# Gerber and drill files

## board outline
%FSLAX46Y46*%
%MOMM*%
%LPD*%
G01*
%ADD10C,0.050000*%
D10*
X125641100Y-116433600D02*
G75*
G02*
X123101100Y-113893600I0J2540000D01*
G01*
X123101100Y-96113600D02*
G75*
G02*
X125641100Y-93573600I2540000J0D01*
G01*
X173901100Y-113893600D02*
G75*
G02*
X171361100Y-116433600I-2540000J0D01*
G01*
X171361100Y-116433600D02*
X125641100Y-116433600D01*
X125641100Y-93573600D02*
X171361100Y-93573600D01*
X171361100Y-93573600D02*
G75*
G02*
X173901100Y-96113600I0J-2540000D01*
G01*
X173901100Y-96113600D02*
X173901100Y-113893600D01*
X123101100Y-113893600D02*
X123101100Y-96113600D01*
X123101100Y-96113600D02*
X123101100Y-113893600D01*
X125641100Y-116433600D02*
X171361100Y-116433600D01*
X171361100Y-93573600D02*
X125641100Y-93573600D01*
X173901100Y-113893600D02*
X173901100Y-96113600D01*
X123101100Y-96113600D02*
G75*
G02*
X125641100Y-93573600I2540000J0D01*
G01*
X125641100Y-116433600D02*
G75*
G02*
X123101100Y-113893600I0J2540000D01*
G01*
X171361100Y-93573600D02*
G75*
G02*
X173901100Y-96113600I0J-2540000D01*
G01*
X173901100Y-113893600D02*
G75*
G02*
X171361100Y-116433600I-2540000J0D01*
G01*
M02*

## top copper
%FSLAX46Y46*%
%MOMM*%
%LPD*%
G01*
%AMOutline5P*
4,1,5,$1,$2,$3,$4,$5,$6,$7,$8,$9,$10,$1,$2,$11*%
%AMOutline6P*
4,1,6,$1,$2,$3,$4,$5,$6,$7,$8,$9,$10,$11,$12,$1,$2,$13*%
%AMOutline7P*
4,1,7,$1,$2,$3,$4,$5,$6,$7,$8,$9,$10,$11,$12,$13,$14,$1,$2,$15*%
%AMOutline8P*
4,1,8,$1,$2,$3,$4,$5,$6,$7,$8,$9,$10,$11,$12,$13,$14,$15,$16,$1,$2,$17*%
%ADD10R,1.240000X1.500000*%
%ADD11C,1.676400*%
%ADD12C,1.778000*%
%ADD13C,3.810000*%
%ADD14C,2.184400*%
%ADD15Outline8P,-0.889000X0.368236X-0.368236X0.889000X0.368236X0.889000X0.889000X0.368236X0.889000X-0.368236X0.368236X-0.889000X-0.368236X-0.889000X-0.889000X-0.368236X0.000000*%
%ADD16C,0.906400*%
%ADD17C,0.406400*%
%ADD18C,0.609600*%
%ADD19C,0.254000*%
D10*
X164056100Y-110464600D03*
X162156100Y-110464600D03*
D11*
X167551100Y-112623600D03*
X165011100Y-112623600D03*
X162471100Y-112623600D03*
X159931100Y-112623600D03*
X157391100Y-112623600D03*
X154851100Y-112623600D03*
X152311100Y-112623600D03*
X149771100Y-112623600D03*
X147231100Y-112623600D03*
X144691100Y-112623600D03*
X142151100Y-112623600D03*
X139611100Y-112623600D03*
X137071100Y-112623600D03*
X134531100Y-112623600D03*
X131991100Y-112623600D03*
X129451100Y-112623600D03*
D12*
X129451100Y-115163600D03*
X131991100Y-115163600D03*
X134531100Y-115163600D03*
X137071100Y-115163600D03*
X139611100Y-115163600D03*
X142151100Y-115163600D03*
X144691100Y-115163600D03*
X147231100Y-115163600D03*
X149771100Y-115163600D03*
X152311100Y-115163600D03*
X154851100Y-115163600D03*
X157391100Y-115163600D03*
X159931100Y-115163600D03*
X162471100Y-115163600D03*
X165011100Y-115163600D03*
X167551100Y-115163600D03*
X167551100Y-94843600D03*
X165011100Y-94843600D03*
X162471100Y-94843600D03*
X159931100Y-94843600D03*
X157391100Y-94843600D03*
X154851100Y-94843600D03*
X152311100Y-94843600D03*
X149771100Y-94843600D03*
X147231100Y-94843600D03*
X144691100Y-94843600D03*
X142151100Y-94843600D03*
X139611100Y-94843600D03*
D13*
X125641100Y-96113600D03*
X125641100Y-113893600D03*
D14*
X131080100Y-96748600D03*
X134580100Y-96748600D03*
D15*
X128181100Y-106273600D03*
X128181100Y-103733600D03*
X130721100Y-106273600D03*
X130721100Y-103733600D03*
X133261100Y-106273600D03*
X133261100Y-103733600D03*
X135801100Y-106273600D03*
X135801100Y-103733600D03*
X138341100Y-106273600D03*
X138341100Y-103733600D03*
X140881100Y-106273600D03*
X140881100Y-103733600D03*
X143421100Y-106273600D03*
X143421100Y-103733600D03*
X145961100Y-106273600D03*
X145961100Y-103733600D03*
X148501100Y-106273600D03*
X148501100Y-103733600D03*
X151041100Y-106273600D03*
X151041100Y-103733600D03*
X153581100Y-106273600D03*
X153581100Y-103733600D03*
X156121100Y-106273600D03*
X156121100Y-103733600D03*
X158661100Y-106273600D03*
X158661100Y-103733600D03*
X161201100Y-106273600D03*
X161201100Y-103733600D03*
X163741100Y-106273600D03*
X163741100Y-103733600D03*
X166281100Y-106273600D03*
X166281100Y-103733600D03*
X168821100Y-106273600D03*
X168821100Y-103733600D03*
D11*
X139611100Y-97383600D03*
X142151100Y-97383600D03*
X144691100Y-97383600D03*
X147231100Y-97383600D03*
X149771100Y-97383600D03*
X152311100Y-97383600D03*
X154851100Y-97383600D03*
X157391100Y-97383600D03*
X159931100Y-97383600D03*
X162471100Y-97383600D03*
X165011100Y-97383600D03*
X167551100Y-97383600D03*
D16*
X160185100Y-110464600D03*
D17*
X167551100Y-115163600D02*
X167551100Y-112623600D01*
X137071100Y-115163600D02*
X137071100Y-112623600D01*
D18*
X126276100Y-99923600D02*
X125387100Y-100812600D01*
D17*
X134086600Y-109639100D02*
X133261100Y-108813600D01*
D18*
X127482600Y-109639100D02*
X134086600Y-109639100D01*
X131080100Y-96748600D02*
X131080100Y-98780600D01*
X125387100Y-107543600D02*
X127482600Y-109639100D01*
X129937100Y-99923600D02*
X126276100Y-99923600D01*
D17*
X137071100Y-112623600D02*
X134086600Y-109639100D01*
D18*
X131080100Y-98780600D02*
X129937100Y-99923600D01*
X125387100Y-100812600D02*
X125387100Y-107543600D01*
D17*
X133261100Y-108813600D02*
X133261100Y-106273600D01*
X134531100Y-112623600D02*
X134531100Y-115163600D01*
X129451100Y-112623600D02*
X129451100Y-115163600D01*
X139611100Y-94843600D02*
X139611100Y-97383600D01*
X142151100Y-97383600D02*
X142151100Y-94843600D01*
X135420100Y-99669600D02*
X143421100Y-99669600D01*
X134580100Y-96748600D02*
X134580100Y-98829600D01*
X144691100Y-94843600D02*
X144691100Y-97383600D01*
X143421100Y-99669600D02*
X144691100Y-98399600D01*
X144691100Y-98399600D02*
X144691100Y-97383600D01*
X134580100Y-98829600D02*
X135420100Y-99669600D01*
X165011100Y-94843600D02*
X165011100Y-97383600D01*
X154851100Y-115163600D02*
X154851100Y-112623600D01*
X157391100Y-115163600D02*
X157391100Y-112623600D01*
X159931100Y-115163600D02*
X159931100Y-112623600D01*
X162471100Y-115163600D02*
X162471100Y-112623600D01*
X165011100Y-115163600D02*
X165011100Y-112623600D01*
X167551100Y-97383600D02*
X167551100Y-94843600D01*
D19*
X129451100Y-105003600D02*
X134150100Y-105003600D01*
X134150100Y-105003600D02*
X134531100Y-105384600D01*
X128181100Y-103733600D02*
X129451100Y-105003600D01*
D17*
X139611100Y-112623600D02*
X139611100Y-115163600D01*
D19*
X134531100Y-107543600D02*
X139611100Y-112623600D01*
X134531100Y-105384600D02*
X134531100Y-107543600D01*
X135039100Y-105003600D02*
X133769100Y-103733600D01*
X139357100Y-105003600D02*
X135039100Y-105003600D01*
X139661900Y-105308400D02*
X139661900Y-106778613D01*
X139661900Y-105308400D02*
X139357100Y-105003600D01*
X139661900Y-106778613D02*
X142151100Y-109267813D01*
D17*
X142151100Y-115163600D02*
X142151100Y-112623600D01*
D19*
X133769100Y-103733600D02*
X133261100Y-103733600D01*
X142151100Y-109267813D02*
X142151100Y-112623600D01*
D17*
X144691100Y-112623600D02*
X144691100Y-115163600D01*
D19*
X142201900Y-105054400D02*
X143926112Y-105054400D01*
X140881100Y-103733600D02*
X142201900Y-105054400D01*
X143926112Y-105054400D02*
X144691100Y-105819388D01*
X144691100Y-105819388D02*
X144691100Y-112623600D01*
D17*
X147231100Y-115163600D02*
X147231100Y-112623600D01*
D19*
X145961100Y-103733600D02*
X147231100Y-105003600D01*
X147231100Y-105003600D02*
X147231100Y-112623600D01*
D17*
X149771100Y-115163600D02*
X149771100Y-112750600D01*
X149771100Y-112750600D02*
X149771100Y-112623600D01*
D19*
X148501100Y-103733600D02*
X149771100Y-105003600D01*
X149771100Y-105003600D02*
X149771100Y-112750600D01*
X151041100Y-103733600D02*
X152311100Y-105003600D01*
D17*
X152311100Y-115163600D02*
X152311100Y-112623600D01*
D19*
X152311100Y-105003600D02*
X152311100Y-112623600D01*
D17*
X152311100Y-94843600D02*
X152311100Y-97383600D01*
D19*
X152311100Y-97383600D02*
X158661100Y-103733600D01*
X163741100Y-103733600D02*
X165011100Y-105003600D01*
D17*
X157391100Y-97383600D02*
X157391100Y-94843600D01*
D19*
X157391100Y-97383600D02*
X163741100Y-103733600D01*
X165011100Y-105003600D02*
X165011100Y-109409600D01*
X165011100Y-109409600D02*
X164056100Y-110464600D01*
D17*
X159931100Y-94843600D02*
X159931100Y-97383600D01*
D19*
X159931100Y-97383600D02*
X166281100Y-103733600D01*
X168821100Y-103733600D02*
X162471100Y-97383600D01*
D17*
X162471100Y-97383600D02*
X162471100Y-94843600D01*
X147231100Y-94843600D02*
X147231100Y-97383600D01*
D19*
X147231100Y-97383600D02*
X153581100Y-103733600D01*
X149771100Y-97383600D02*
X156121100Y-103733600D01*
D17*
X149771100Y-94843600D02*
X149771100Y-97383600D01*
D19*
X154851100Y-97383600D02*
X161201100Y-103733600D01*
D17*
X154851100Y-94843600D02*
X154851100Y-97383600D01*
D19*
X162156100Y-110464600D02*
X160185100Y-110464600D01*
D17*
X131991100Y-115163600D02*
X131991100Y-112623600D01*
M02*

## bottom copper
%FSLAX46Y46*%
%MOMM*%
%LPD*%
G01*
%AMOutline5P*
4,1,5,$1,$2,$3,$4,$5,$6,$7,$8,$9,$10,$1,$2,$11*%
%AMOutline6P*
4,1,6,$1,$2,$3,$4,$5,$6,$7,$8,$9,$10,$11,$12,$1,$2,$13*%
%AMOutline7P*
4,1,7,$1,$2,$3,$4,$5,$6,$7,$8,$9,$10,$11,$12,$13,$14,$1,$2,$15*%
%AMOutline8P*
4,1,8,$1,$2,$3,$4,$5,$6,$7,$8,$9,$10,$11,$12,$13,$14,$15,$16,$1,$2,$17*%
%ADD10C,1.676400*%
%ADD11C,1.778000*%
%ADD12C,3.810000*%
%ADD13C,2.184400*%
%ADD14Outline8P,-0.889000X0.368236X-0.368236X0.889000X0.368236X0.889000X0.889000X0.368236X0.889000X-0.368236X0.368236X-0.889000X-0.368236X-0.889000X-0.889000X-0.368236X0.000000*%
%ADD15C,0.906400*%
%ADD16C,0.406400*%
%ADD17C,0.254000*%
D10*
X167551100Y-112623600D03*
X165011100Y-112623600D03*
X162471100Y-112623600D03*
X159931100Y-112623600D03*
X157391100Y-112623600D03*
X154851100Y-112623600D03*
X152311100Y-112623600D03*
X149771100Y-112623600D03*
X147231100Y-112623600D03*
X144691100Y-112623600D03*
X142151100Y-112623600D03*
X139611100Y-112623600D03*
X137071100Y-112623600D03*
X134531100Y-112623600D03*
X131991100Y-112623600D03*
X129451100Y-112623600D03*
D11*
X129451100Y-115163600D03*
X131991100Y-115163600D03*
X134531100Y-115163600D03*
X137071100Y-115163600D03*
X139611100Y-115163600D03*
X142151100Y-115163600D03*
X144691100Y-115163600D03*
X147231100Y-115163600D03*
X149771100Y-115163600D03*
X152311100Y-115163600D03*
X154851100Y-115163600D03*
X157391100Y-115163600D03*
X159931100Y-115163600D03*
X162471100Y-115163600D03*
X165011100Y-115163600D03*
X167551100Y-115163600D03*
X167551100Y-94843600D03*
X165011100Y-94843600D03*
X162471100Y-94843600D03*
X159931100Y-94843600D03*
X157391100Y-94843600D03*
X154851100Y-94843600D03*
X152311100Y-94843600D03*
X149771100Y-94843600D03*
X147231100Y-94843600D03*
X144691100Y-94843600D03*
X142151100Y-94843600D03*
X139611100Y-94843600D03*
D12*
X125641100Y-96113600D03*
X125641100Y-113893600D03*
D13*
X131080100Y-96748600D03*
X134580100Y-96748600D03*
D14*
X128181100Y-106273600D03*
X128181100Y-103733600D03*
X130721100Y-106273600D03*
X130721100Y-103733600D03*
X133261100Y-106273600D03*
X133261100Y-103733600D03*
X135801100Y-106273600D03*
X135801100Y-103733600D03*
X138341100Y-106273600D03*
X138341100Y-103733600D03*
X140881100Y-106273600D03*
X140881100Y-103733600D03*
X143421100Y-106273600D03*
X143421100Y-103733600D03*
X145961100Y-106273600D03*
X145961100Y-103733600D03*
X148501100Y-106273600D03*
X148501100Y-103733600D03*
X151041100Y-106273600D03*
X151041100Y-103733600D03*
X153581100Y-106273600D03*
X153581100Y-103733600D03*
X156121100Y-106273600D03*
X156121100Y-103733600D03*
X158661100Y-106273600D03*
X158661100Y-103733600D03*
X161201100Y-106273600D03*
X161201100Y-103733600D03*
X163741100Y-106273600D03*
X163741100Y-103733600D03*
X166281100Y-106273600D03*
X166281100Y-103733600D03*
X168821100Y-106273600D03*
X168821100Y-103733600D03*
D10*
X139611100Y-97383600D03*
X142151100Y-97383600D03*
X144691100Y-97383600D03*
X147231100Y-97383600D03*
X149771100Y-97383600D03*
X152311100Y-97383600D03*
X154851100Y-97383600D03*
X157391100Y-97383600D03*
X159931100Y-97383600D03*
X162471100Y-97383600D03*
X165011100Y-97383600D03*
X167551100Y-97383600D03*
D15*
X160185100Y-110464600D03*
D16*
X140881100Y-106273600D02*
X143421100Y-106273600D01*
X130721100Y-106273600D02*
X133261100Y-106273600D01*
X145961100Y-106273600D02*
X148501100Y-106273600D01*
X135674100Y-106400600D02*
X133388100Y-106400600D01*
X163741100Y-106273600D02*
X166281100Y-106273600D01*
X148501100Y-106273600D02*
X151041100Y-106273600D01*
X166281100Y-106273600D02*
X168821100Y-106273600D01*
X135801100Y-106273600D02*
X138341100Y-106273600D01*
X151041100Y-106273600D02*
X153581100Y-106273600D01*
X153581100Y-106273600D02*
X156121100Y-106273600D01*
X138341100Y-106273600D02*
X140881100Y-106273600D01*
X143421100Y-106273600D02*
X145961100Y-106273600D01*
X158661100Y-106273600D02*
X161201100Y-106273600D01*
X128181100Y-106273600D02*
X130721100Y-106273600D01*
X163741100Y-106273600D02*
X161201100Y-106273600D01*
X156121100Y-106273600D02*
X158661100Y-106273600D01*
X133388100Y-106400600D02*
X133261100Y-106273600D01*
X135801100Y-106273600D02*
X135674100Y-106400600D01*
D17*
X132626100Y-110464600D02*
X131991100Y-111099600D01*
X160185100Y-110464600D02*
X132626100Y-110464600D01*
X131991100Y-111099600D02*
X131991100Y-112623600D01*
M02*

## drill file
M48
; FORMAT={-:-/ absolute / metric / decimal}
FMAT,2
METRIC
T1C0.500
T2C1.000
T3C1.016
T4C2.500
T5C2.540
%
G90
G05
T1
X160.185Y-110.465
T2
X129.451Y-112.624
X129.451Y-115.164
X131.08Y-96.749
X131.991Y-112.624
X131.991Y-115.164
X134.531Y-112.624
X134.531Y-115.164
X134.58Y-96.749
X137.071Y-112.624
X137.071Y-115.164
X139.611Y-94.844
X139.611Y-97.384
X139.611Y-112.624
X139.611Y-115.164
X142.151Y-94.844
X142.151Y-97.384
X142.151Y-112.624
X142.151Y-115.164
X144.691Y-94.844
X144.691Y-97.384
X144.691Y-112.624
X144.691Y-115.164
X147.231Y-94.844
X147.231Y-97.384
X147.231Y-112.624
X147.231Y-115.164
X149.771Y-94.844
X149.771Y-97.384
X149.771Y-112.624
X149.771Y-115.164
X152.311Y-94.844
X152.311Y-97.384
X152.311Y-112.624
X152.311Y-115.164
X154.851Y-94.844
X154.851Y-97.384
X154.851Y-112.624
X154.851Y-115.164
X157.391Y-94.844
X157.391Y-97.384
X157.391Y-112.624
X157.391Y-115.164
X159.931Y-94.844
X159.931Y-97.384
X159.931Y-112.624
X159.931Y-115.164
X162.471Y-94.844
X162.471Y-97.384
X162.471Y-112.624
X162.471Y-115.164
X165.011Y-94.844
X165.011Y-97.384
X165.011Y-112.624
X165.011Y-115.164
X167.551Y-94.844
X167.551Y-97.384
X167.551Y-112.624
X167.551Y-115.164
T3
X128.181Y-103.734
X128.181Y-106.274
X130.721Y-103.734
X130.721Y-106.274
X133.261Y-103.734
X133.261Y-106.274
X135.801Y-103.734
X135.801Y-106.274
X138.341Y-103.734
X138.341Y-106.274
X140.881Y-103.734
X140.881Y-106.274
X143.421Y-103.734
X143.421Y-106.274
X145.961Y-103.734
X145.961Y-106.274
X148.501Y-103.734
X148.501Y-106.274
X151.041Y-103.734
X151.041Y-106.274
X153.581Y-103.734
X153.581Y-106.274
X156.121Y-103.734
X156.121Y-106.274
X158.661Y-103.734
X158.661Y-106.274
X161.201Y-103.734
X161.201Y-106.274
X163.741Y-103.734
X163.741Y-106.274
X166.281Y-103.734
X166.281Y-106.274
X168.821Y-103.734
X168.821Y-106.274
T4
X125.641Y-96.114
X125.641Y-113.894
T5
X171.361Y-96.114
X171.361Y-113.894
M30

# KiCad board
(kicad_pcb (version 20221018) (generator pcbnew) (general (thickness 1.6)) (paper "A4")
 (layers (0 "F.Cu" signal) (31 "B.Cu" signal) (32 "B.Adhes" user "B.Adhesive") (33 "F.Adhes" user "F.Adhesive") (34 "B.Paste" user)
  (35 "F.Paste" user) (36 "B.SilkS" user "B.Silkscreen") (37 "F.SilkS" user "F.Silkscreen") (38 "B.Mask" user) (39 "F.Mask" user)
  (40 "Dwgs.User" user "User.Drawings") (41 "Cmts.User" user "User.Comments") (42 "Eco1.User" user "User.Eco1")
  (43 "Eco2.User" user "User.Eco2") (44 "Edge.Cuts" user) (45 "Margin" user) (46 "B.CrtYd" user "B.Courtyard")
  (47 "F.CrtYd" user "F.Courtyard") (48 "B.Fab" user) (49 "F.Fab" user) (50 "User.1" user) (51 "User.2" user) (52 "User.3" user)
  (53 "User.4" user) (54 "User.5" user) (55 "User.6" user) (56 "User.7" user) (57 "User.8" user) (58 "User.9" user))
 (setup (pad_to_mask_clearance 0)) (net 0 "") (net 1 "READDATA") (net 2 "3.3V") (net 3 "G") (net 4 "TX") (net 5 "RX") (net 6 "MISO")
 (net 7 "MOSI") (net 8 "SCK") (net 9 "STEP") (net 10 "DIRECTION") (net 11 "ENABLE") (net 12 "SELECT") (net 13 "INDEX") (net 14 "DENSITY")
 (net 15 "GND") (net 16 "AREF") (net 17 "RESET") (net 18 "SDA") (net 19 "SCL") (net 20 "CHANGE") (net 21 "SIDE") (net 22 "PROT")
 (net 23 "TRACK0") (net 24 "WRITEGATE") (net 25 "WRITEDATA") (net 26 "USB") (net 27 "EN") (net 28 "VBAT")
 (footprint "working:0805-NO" (layer "F.Cu") (at 163.1061 110.4646 180)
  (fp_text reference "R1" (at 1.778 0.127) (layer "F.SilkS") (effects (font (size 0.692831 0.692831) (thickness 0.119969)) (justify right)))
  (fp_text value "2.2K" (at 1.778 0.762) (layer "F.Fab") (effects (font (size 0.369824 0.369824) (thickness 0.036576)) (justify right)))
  (pad "1" smd rect (at -0.95 0 180) (size 1.24 1.5) (layers "F.Cu" "F.Paste" "F.Mask") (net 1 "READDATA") (solder_mask_margin 0.0508)
   (thermal_bridge_angle 45))
  (pad "2" smd rect (at 0.95 0 180) (size 1.24 1.5) (layers "F.Cu" "F.Paste" "F.Mask") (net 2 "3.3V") (solder_mask_margin 0.0508)
   (thermal_bridge_angle 45)))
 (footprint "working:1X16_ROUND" (layer "F.Cu") (at 148.5011 112.6236 180)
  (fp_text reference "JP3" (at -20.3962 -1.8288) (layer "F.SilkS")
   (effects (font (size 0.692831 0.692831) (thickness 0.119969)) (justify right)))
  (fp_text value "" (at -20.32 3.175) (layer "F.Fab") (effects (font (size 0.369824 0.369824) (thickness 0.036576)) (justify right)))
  (pad "1" thru_hole circle (at -19.05 0 270) (size 1.6764 1.6764) (drill 1) (layers "*.Cu" "*.Mask") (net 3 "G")
   (solder_mask_margin 0.0508))
  (pad "2" thru_hole circle (at -16.51 0 270) (size 1.6764 1.6764) (drill 1) (layers "*.Cu" "*.Mask") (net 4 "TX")
   (solder_mask_margin 0.0508))
  (pad "3" thru_hole circle (at -13.97 0 270) (size 1.6764 1.6764) (drill 1) (layers "*.Cu" "*.Mask") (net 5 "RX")
   (solder_mask_margin 0.0508))
  (pad "4" thru_hole circle (at -11.43 0 270) (size 1.6764 1.6764) (drill 1) (layers "*.Cu" "*.Mask") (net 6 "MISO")
   (solder_mask_margin 0.0508))
  (pad "5" thru_hole circle (at -8.89 0 270) (size 1.6764 1.6764) (drill 1) (layers "*.Cu" "*.Mask") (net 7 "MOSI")
   (solder_mask_margin 0.0508))
  (pad "6" thru_hole circle (at -6.35 0 270) (size 1.6764 1.6764) (drill 1) (layers "*.Cu" "*.Mask") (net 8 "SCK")
   (solder_mask_margin 0.0508))
  (pad "7" thru_hole circle (at -3.81 0 270) (size 1.6764 1.6764) (drill 1) (layers "*.Cu" "*.Mask") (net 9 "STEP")
   (solder_mask_margin 0.0508))
  (pad "8" thru_hole circle (at -1.27 0 270) (size 1.6764 1.6764) (drill 1) (layers "*.Cu" "*.Mask") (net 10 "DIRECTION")
   (solder_mask_margin 0.0508))
  (pad "9" thru_hole circle (at 1.27 0 270) (size 1.6764 1.6764) (drill 1) (layers "*.Cu" "*.Mask") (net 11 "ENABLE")
   (solder_mask_margin 0.0508))
  (pad "10" thru_hole circle (at 3.81 0 270) (size 1.6764 1.6764) (drill 1) (layers "*.Cu" "*.Mask") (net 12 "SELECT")
   (solder_mask_margin 0.0508))
  (pad "11" thru_hole circle (at 6.35 0 270) (size 1.6764 1.6764) (drill 1) (layers "*.Cu" "*.Mask") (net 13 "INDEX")
   (solder_mask_margin 0.0508))
  (pad "12" thru_hole circle (at 8.89 0 270) (size 1.6764 1.6764) (drill 1) (layers "*.Cu" "*.Mask") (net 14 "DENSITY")
   (solder_mask_margin 0.0508))
  (pad "13" thru_hole circle (at 11.43 0 270) (size 1.6764 1.6764) (drill 1) (layers "*.Cu" "*.Mask") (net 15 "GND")
   (solder_mask_margin 0.0508))
  (pad "14" thru_hole circle (at 13.97 0 270) (size 1.6764 1.6764) (drill 1) (layers "*.Cu" "*.Mask") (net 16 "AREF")
   (solder_mask_margin 0.0508))
  (pad "15" thru_hole circle (at 16.51 0 270) (size 1.6764 1.6764) (drill 1) (layers "*.Cu" "*.Mask") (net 2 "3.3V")
   (solder_mask_margin 0.0508))
  (pad "16" thru_hole circle (at 19.05 0 270) (size 1.6764 1.6764) (drill 1) (layers "*.Cu" "*.Mask") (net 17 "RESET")
   (solder_mask_margin 0.0508)))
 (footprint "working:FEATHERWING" (layer "F.Cu") (at 123.1011 116.4336)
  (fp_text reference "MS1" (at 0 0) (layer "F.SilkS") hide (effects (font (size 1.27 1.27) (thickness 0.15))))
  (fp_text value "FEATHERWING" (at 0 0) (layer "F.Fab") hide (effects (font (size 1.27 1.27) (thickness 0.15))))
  (fp_line (start 0 -20.32) (end 0 -2.54) (stroke (width 0.05) (type solid)) (layer "Edge.Cuts"))
  (fp_line (start 2.54 0) (end 48.26 0) (stroke (width 0.05) (type solid)) (layer "Edge.Cuts"))
  (fp_line (start 48.26 -22.86) (end 2.54 -22.86) (stroke (width 0.05) (type solid)) (layer "Edge.Cuts"))
  (fp_line (start 50.8 -2.54) (end 50.8 -20.32) (stroke (width 0.05) (type solid)) (layer "Edge.Cuts"))
  (fp_arc (start 0 -20.32) (mid 0.743949 -22.116051) (end 2.54 -22.86) (stroke (width 0.05) (type solid)) (layer "Edge.Cuts"))
  (fp_arc (start 2.54 0) (mid 0.743949 -0.743949) (end 0 -2.54) (stroke (width 0.05) (type solid)) (layer "Edge.Cuts"))
  (fp_arc (start 48.26 -22.86) (mid 50.056051 -22.116051) (end 50.8 -20.32) (stroke (width 0.05) (type solid)) (layer "Edge.Cuts"))
  (fp_arc (start 50.8 -2.54) (mid 50.056051 -0.743949) (end 48.26 0) (stroke (width 0.05) (type solid)) (layer "Edge.Cuts"))
  (pad "" np_thru_hole circle (at 48.26 -20.32) (size 2.54 2.54) (drill 2.54) (layers "*.Cu" "*.Mask"))
  (pad "" np_thru_hole circle (at 48.26 -2.54) (size 2.54 2.54) (drill 2.54) (layers "*.Cu" "*.Mask"))
  (pad "1" thru_hole circle (at 6.35 -1.27) (size 1.778 1.778) (drill 1) (layers "*.Cu" "*.Mask") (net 17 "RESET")
   (solder_mask_margin 0.0508))
  (pad "2" thru_hole circle (at 8.89 -1.27) (size 1.778 1.778) (drill 1) (layers "*.Cu" "*.Mask") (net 2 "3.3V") (solder_mask_margin 0.0508))
  (pad "3" thru_hole circle (at 11.43 -1.27) (size 1.778 1.778) (drill 1) (layers "*.Cu" "*.Mask") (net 16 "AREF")
   (solder_mask_margin 0.0508))
  (pad "4" thru_hole circle (at 13.97 -1.27) (size 1.778 1.778) (drill 1) (layers "*.Cu" "*.Mask") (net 15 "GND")
   (solder_mask_margin 0.0508))
  (pad "5" thru_hole circle (at 16.51 -1.27) (size 1.778 1.778) (drill 1) (layers "*.Cu" "*.Mask") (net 14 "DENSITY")
   (solder_mask_margin 0.0508))
  (pad "6" thru_hole circle (at 19.05 -1.27) (size 1.778 1.778) (drill 1) (layers "*.Cu" "*.Mask") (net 13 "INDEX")
   (solder_mask_margin 0.0508))
  (pad "7" thru_hole circle (at 21.59 -1.27) (size 1.778 1.778) (drill 1) (layers "*.Cu" "*.Mask") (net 12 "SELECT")
   (solder_mask_margin 0.0508))
  (pad "8" thru_hole circle (at 24.13 -1.27) (size 1.778 1.778) (drill 1) (layers "*.Cu" "*.Mask") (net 11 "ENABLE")
   (solder_mask_margin 0.0508))
  (pad "9" thru_hole circle (at 26.67 -1.27) (size 1.778 1.778) (drill 1) (layers "*.Cu" "*.Mask") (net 10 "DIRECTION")
   (solder_mask_margin 0.0508))
  (pad "10" thru_hole circle (at 29.21 -1.27) (size 1.778 1.778) (drill 1) (layers "*.Cu" "*.Mask") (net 9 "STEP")
   (solder_mask_margin 0.0508))
  (pad "11" thru_hole circle (at 31.75 -1.27) (size 1.778 1.778) (drill 1) (layers "*.Cu" "*.Mask") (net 8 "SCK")
   (solder_mask_margin 0.0508))
  (pad "12" thru_hole circle (at 34.29 -1.27) (size 1.778 1.778) (drill 1) (layers "*.Cu" "*.Mask") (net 7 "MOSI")
   (solder_mask_margin 0.0508))
  (pad "13" thru_hole circle (at 36.83 -1.27) (size 1.778 1.778) (drill 1) (layers "*.Cu" "*.Mask") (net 6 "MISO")
   (solder_mask_margin 0.0508))
  (pad "14" thru_hole circle (at 39.37 -1.27) (size 1.778 1.778) (drill 1) (layers "*.Cu" "*.Mask") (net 5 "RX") (solder_mask_margin 0.0508))
  (pad "15" thru_hole circle (at 41.91 -1.27) (size 1.778 1.778) (drill 1) (layers "*.Cu" "*.Mask") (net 4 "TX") (solder_mask_margin 0.0508))
  (pad "16" thru_hole circle (at 44.45 -1.27) (size 1.778 1.778) (drill 1) (layers "*.Cu" "*.Mask") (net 3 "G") (solder_mask_margin 0.0508))
  (pad "17" thru_hole circle (at 44.45 -21.59) (size 1.778 1.778) (drill 1) (layers "*.Cu" "*.Mask") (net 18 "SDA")
   (solder_mask_margin 0.0508))
  (pad "18" thru_hole circle (at 41.91 -21.59) (size 1.778 1.778) (drill 1) (layers "*.Cu" "*.Mask") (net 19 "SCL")
   (solder_mask_margin 0.0508))
  (pad "19" thru_hole circle (at 39.37 -21.59) (size 1.778 1.778) (drill 1) (layers "*.Cu" "*.Mask") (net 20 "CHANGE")
   (solder_mask_margin 0.0508))
  (pad "20" thru_hole circle (at 36.83 -21.59) (size 1.778 1.778) (drill 1) (layers "*.Cu" "*.Mask") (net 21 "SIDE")
   (solder_mask_margin 0.0508))
  (pad "21" thru_hole circle (at 34.29 -21.59) (size 1.778 1.778) (drill 1) (layers "*.Cu" "*.Mask") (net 1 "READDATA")
   (solder_mask_margin 0.0508))
  (pad "22" thru_hole circle (at 31.75 -21.59) (size 1.778 1.778) (drill 1) (layers "*.Cu" "*.Mask") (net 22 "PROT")
   (solder_mask_margin 0.0508))
  (pad "23" thru_hole circle (at 29.21 -21.59) (size 1.778 1.778) (drill 1) (layers "*.Cu" "*.Mask") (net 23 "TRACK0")
   (solder_mask_margin 0.0508))
  (pad "24" thru_hole circle (at 26.67 -21.59) (size 1.778 1.778) (drill 1) (layers "*.Cu" "*.Mask") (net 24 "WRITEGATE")
   (solder_mask_margin 0.0508))
  (pad "25" thru_hole circle (at 24.13 -21.59) (size 1.778 1.778) (drill 1) (layers "*.Cu" "*.Mask") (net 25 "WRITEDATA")
   (solder_mask_margin 0.0508))
  (pad "26" thru_hole circle (at 21.59 -21.59) (size 1.778 1.778) (drill 1) (layers "*.Cu" "*.Mask") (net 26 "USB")
   (solder_mask_margin 0.0508))
  (pad "27" thru_hole circle (at 19.05 -21.59) (size 1.778 1.778) (drill 1) (layers "*.Cu" "*.Mask") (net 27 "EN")
   (solder_mask_margin 0.0508))
  (pad "28" thru_hole circle (at 16.51 -21.59) (size 1.778 1.778) (drill 1) (layers "*.Cu" "*.Mask") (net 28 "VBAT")
   (solder_mask_margin 0.0508))
  (pad "P$1" thru_hole circle (at 2.54 -20.32) (size 3.81 3.81) (drill 2.5) (layers "*.Cu" "*.Mask") (solder_mask_margin 0.0508))
  (pad "P$2" thru_hole circle (at 2.54 -2.54) (size 3.81 3.81) (drill 2.5) (layers "*.Cu" "*.Mask") (solder_mask_margin 0.0508)))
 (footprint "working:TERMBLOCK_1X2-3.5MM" (layer "F.Cu") (at 132.8801 96.7486 180)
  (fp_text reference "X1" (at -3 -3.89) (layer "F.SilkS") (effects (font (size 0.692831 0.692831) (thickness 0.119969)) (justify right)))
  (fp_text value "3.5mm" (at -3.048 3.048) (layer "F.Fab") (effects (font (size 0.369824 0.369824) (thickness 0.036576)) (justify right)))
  (pad "1" thru_hole circle (at 1.8 0 180) (size 2.1844 2.1844) (drill 1) (layers "*.Cu" "*.Mask") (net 15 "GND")
   (solder_mask_margin 0.0508))
  (pad "2" thru_hole circle (at -1.7 0 180) (size 2.1844 2.1844) (drill 1) (layers "*.Cu" "*.Mask") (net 26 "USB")
   (solder_mask_margin 0.0508)))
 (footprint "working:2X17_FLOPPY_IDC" (layer "F.Cu") (at 148.5011 105.0036 90)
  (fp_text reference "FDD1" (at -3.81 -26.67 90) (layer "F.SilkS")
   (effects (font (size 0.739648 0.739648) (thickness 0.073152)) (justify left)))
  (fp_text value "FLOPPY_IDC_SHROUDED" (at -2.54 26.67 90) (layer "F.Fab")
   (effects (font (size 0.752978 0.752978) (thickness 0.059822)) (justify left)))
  (pad "1" thru_hole roundrect (at -1.27 -20.32) (size 1.778 1.778) (drill 1.016) (layers "*.Cu" "*.Mask") (roundrect_rratio 0.25)
   (chamfer_ratio 0.2928932188) (chamfer top_left top_right bottom_left bottom_right) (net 15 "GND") (solder_mask_margin 0.0508)
   (thermal_bridge_angle 45))
  (pad "2" thru_hole roundrect (at 1.27 -20.32) (size 1.778 1.778) (drill 1.016) (layers "*.Cu" "*.Mask") (roundrect_rratio 0.25)
   (chamfer_ratio 0.2928932188) (chamfer top_left top_right bottom_left bottom_right) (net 14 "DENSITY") (solder_mask_margin 0.0508)
   (thermal_bridge_angle 45))
  (pad "3" thru_hole roundrect (at -1.27 -17.78) (size 1.778 1.778) (drill 1.016) (layers "*.Cu" "*.Mask") (roundrect_rratio 0.25)
   (chamfer_ratio 0.2928932188) (chamfer top_left top_right bottom_left bottom_right) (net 15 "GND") (solder_mask_margin 0.0508)
   (thermal_bridge_angle 45))
  (pad "4" thru_hole roundrect (at 1.27 -17.78) (size 1.778 1.778) (drill 1.016) (layers "*.Cu" "*.Mask") (roundrect_rratio 0.25)
   (chamfer_ratio 0.2928932188) (chamfer top_left top_right bottom_left bottom_right) (solder_mask_margin 0.0508) (thermal_bridge_angle 45))
  (pad "5" thru_hole roundrect (at -1.27 -15.24) (size 1.778 1.778) (drill 1.016) (layers "*.Cu" "*.Mask") (roundrect_rratio 0.25)
   (chamfer_ratio 0.2928932188) (chamfer top_left top_right bottom_left bottom_right) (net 15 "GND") (solder_mask_margin 0.0508)
   (thermal_bridge_angle 45))
  (pad "6" thru_hole roundrect (at 1.27 -15.24) (size 1.778 1.778) (drill 1.016) (layers "*.Cu" "*.Mask") (roundrect_rratio 0.25)
   (chamfer_ratio 0.2928932188) (chamfer top_left top_right bottom_left bottom_right) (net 13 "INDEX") (solder_mask_margin 0.0508)
   (thermal_bridge_angle 45))
  (pad "7" thru_hole roundrect (at -1.27 -12.7) (size 1.778 1.778) (drill 1.016) (layers "*.Cu" "*.Mask") (roundrect_rratio 0.25)
   (chamfer_ratio 0.2928932188) (chamfer top_left top_right bottom_left bottom_right) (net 15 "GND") (solder_mask_margin 0.0508)
   (thermal_bridge_angle 45))
  (pad "8" thru_hole roundrect (at 1.27 -12.7) (size 1.778 1.778) (drill 1.016) (layers "*.Cu" "*.Mask") (roundrect_rratio 0.25)
   (chamfer_ratio 0.2928932188) (chamfer top_left top_right bottom_left bottom_right) (solder_mask_margin 0.0508) (thermal_bridge_angle 45))
  (pad "9" thru_hole roundrect (at -1.27 -10.16) (size 1.778 1.778) (drill 1.016) (layers "*.Cu" "*.Mask") (roundrect_rratio 0.25)
   (chamfer_ratio 0.2928932188) (chamfer top_left top_right bottom_left bottom_right) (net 15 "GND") (solder_mask_margin 0.0508)
   (thermal_bridge_angle 45))
  (pad "10" thru_hole roundrect (at 1.27 -10.16) (size 1.778 1.778) (drill 1.016) (layers "*.Cu" "*.Mask") (roundrect_rratio 0.25)
   (chamfer_ratio 0.2928932188) (chamfer top_left top_right bottom_left bottom_right) (solder_mask_margin 0.0508) (thermal_bridge_angle 45))
  (pad "11" thru_hole roundrect (at -1.27 -7.62) (size 1.778 1.778) (drill 1.016) (layers "*.Cu" "*.Mask") (roundrect_rratio 0.25)
   (chamfer_ratio 0.2928932188) (chamfer top_left top_right bottom_left bottom_right) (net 15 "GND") (solder_mask_margin 0.0508)
   (thermal_bridge_angle 45))
  (pad "12" thru_hole roundrect (at 1.27 -7.62) (size 1.778 1.778) (drill 1.016) (layers "*.Cu" "*.Mask") (roundrect_rratio 0.25)
   (chamfer_ratio 0.2928932188) (chamfer top_left top_right bottom_left bottom_right) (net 12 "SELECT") (solder_mask_margin 0.0508)
   (thermal_bridge_angle 45))
  (pad "13" thru_hole roundrect (at -1.27 -5.08) (size 1.778 1.778) (drill 1.016) (layers "*.Cu" "*.Mask") (roundrect_rratio 0.25)
   (chamfer_ratio 0.2928932188) (chamfer top_left top_right bottom_left bottom_right) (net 15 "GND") (solder_mask_margin 0.0508)
   (thermal_bridge_angle 45))
  (pad "14" thru_hole roundrect (at 1.27 -5.08) (size 1.778 1.778) (drill 1.016) (layers "*.Cu" "*.Mask") (roundrect_rratio 0.25)
   (chamfer_ratio 0.2928932188) (chamfer top_left top_right bottom_left bottom_right) (solder_mask_margin 0.0508) (thermal_bridge_angle 45))
  (pad "15" thru_hole roundrect (at -1.27 -2.54) (size 1.778 1.778) (drill 1.016) (layers "*.Cu" "*.Mask") (roundrect_rratio 0.25)
   (chamfer_ratio 0.2928932188) (chamfer top_left top_right bottom_left bottom_right) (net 15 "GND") (solder_mask_margin 0.0508)
   (thermal_bridge_angle 45))
  (pad "16" thru_hole roundrect (at 1.27 -2.54) (size 1.778 1.778) (drill 1.016) (layers "*.Cu" "*.Mask") (roundrect_rratio 0.25)
   (chamfer_ratio 0.2928932188) (chamfer top_left top_right bottom_left bottom_right) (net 11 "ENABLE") (solder_mask_margin 0.0508)
   (thermal_bridge_angle 45))
  (pad "17" thru_hole roundrect (at -1.27 0) (size 1.778 1.778) (drill 1.016) (layers "*.Cu" "*.Mask") (roundrect_rratio 0.25)
   (chamfer_ratio 0.2928932188) (chamfer top_left top_right bottom_left bottom_right) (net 15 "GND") (solder_mask_margin 0.0508)
   (thermal_bridge_angle 45))
  (pad "18" thru_hole roundrect (at 1.27 0) (size 1.778 1.778) (drill 1.016) (layers "*.Cu" "*.Mask") (roundrect_rratio 0.25)
   (chamfer_ratio 0.2928932188) (chamfer top_left top_right bottom_left bottom_right) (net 10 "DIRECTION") (solder_mask_margin 0.0508)
   (thermal_bridge_angle 45))
  (pad "19" thru_hole roundrect (at -1.27 2.54) (size 1.778 1.778) (drill 1.016) (layers "*.Cu" "*.Mask") (roundrect_rratio 0.25)
   (chamfer_ratio 0.2928932188) (chamfer top_left top_right bottom_left bottom_right) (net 15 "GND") (solder_mask_margin 0.0508)
   (thermal_bridge_angle 45))
  (pad "20" thru_hole roundrect (at 1.27 2.54) (size 1.778 1.778) (drill 1.016) (layers "*.Cu" "*.Mask") (roundrect_rratio 0.25)
   (chamfer_ratio 0.2928932188) (chamfer top_left top_right bottom_left bottom_right) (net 9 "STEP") (solder_mask_margin 0.0508)
   (thermal_bridge_angle 45))
  (pad "21" thru_hole roundrect (at -1.27 5.08) (size 1.778 1.778) (drill 1.016) (layers "*.Cu" "*.Mask") (roundrect_rratio 0.25)
   (chamfer_ratio 0.2928932188) (chamfer top_left top_right bottom_left bottom_right) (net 15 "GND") (solder_mask_margin 0.0508)
   (thermal_bridge_angle 45))
  (pad "22" thru_hole roundrect (at 1.27 5.08) (size 1.778 1.778) (drill 1.016) (layers "*.Cu" "*.Mask") (roundrect_rratio 0.25)
   (chamfer_ratio 0.2928932188) (chamfer top_left top_right bottom_left bottom_right) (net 25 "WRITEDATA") (solder_mask_margin 0.0508)
   (thermal_bridge_angle 45))
  (pad "23" thru_hole roundrect (at -1.27 7.62) (size 1.778 1.778) (drill 1.016) (layers "*.Cu" "*.Mask") (roundrect_rratio 0.25)
   (chamfer_ratio 0.2928932188) (chamfer top_left top_right bottom_left bottom_right) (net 15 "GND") (solder_mask_margin 0.0508)
   (thermal_bridge_angle 45))
  (pad "24" thru_hole roundrect (at 1.27 7.62) (size 1.778 1.778) (drill 1.016) (layers "*.Cu" "*.Mask") (roundrect_rratio 0.25)
   (chamfer_ratio 0.2928932188) (chamfer top_left top_right bottom_left bottom_right) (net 24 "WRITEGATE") (solder_mask_margin 0.0508)
   (thermal_bridge_angle 45))
  (pad "25" thru_hole roundrect (at -1.27 10.16) (size 1.778 1.778) (drill 1.016) (layers "*.Cu" "*.Mask") (roundrect_rratio 0.25)
   (chamfer_ratio 0.2928932188) (chamfer top_left top_right bottom_left bottom_right) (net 15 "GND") (solder_mask_margin 0.0508)
   (thermal_bridge_angle 45))
  (pad "26" thru_hole roundrect (at 1.27 10.16) (size 1.778 1.778) (drill 1.016) (layers "*.Cu" "*.Mask") (roundrect_rratio 0.25)
   (chamfer_ratio 0.2928932188) (chamfer top_left top_right bottom_left bottom_right) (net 23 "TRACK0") (solder_mask_margin 0.0508)
   (thermal_bridge_angle 45))
  (pad "27" thru_hole roundrect (at -1.27 12.7) (size 1.778 1.778) (drill 1.016) (layers "*.Cu" "*.Mask") (roundrect_rratio 0.25)
   (chamfer_ratio 0.2928932188) (chamfer top_left top_right bottom_left bottom_right) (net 15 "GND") (solder_mask_margin 0.0508)
   (thermal_bridge_angle 45))
  (pad "28" thru_hole roundrect (at 1.27 12.7) (size 1.778 1.778) (drill 1.016) (layers "*.Cu" "*.Mask") (roundrect_rratio 0.25)
   (chamfer_ratio 0.2928932188) (chamfer top_left top_right bottom_left bottom_right) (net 22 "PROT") (solder_mask_margin 0.0508)
   (thermal_bridge_angle 45))
  (pad "29" thru_hole roundrect (at -1.27 15.24) (size 1.778 1.778) (drill 1.016) (layers "*.Cu" "*.Mask") (roundrect_rratio 0.25)
   (chamfer_ratio 0.2928932188) (chamfer top_left top_right bottom_left bottom_right) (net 15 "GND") (solder_mask_margin 0.0508)
   (thermal_bridge_angle 45))
  (pad "30" thru_hole roundrect (at 1.27 15.24) (size 1.778 1.778) (drill 1.016) (layers "*.Cu" "*.Mask") (roundrect_rratio 0.25)
   (chamfer_ratio 0.2928932188) (chamfer top_left top_right bottom_left bottom_right) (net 1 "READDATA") (solder_mask_margin 0.0508)
   (thermal_bridge_angle 45))
  (pad "31" thru_hole roundrect (at -1.27 17.78) (size 1.778 1.778) (drill 1.016) (layers "*.Cu" "*.Mask") (roundrect_rratio 0.25)
   (chamfer_ratio 0.2928932188) (chamfer top_left top_right bottom_left bottom_right) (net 15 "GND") (solder_mask_margin 0.0508)
   (thermal_bridge_angle 45))
  (pad "32" thru_hole roundrect (at 1.27 17.78) (size 1.778 1.778) (drill 1.016) (layers "*.Cu" "*.Mask") (roundrect_rratio 0.25)
   (chamfer_ratio 0.2928932188) (chamfer top_left top_right bottom_left bottom_right) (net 21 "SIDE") (solder_mask_margin 0.0508)
   (thermal_bridge_angle 45))
  (pad "33" thru_hole roundrect (at -1.27 20.32) (size 1.778 1.778) (drill 1.016) (layers "*.Cu" "*.Mask") (roundrect_rratio 0.25)
   (chamfer_ratio 0.2928932188) (chamfer top_left top_right bottom_left bottom_right) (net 15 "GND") (solder_mask_margin 0.0508)
   (thermal_bridge_angle 45))
  (pad "34" thru_hole roundrect (at 1.27 20.32) (size 1.778 1.778) (drill 1.016) (layers "*.Cu" "*.Mask") (roundrect_rratio 0.25)
   (chamfer_ratio 0.2928932188) (chamfer top_left top_right bottom_left bottom_right) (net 20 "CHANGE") (solder_mask_margin 0.0508)
   (thermal_bridge_angle 45)))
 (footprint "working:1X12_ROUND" (layer "F.Cu") (at 153.5811 97.3836)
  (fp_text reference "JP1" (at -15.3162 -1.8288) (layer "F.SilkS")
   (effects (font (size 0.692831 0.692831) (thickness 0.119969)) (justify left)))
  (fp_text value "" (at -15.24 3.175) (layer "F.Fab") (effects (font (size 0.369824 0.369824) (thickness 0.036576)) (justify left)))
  (pad "1" thru_hole circle (at -13.97 0 90) (size 1.6764 1.6764) (drill 1) (layers "*.Cu" "*.Mask") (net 28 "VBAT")
   (solder_mask_margin 0.0508))
  (pad "2" thru_hole circle (at -11.43 0 90) (size 1.6764 1.6764) (drill 1) (layers "*.Cu" "*.Mask") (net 27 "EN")
   (solder_mask_margin 0.0508))
  (pad "3" thru_hole circle (at -8.89 0 90) (size 1.6764 1.6764) (drill 1) (layers "*.Cu" "*.Mask") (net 26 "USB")
   (solder_mask_margin 0.0508))
  (pad "4" thru_hole circle (at -6.35 0 90) (size 1.6764 1.6764) (drill 1) (layers "*.Cu" "*.Mask") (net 25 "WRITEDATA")
   (solder_mask_margin 0.0508))
  (pad "5" thru_hole circle (at -3.81 0 90) (size 1.6764 1.6764) (drill 1) (layers "*.Cu" "*.Mask") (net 24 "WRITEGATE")
   (solder_mask_margin 0.0508))
  (pad "6" thru_hole circle (at -1.27 0 90) (size 1.6764 1.6764) (drill 1) (layers "*.Cu" "*.Mask") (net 23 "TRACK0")
   (solder_mask_margin 0.0508))
  (pad "7" thru_hole circle (at 1.27 0 90) (size 1.6764 1.6764) (drill 1) (layers "*.Cu" "*.Mask") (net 22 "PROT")
   (solder_mask_margin 0.0508))
  (pad "8" thru_hole circle (at 3.81 0 90) (size 1.6764 1.6764) (drill 1) (layers "*.Cu" "*.Mask") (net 1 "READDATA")
   (solder_mask_margin 0.0508))
  (pad "9" thru_hole circle (at 6.35 0 90) (size 1.6764 1.6764) (drill 1) (layers "*.Cu" "*.Mask") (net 21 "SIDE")
   (solder_mask_margin 0.0508))
  (pad "10" thru_hole circle (at 8.89 0 90) (size 1.6764 1.6764) (drill 1) (layers "*.Cu" "*.Mask") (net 20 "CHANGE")
   (solder_mask_margin 0.0508))
  (pad "11" thru_hole circle (at 11.43 0 90) (size 1.6764 1.6764) (drill 1) (layers "*.Cu" "*.Mask") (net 19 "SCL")
   (solder_mask_margin 0.0508))
  (pad "12" thru_hole circle (at 13.97 0 90) (size 1.6764 1.6764) (drill 1) (layers "*.Cu" "*.Mask") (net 18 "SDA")
   (solder_mask_margin 0.0508)))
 (gr_arc (start 125.6411 116.4336) (mid 123.845049 115.689651) (end 123.1011 113.8936) (stroke (width 0.05) (type solid))
  (layer "Edge.Cuts"))
 (gr_arc (start 123.1011 96.1136) (mid 123.845049 94.317549) (end 125.6411 93.5736) (stroke (width 0.05) (type solid)) (layer "Edge.Cuts"))
 (gr_arc (start 173.9011 113.8936) (mid 173.157151 115.689651) (end 171.3611 116.4336) (stroke (width 0.05) (type solid))
  (layer "Edge.Cuts"))
 (gr_line (start 171.3611 116.4336) (end 125.6411 116.4336) (stroke (width 0.05) (type solid)) (layer "Edge.Cuts"))
 (gr_line (start 125.6411 93.5736) (end 171.3611 93.5736) (stroke (width 0.05) (type solid)) (layer "Edge.Cuts"))
 (gr_arc (start 171.3611 93.5736) (mid 173.157151 94.317549) (end 173.9011 96.1136) (stroke (width 0.05) (type solid)) (layer "Edge.Cuts"))
 (gr_line (start 173.9011 96.1136) (end 173.9011 113.8936) (stroke (width 0.05) (type solid)) (layer "Edge.Cuts"))
 (gr_line (start 123.1011 113.8936) (end 123.1011 96.1136) (stroke (width 0.05) (type solid)) (layer "Edge.Cuts"))
 (segment (start 167.5511 115.1636) (end 167.5511 112.6236) (width 0.4064) (layer "F.Cu") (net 3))
 (segment (start 137.0711 115.1636) (end 137.0711 112.6236) (width 0.4064) (layer "F.Cu") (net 15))
 (segment (start 126.2761 99.9236) (end 125.3871 100.8126) (width 0.6096) (layer "F.Cu") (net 15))
 (segment (start 134.0866 109.6391) (end 133.2611 108.8136) (width 0.4064) (layer "F.Cu") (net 15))
 (segment (start 127.4826 109.6391) (end 134.0866 109.6391) (width 0.6096) (layer "F.Cu") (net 15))
 (segment (start 131.0801 96.7486) (end 131.0801 98.7806) (width 0.6096) (layer "F.Cu") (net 15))
 (segment (start 125.3871 107.5436) (end 127.4826 109.6391) (width 0.6096) (layer "F.Cu") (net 15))
 (segment (start 129.9371 99.9236) (end 126.2761 99.9236) (width 0.6096) (layer "F.Cu") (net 15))
 (segment (start 137.0711 112.6236) (end 134.0866 109.6391) (width 0.4064) (layer "F.Cu") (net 15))
 (segment (start 131.0801 98.7806) (end 129.9371 99.9236) (width 0.6096) (layer "F.Cu") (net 15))
 (segment (start 125.3871 100.8126) (end 125.3871 107.5436) (width 0.6096) (layer "F.Cu") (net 15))
 (segment (start 133.2611 108.8136) (end 133.2611 106.2736) (width 0.4064) (layer "F.Cu") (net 15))
 (segment (start 140.8811 106.2736) (end 143.4211 106.2736) (width 0.4064) (layer "B.Cu") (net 15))
 (segment (start 130.7211 106.2736) (end 133.2611 106.2736) (width 0.4064) (layer "B.Cu") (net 15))
 (segment (start 145.9611 106.2736) (end 148.5011 106.2736) (width 0.4064) (layer "B.Cu") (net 15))
 (segment (start 135.6741 106.4006) (end 133.3881 106.4006) (width 0.4064) (layer "B.Cu") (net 15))
 (segment (start 163.7411 106.2736) (end 166.2811 106.2736) (width 0.4064) (layer "B.Cu") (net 15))
 (segment (start 148.5011 106.2736) (end 151.0411 106.2736) (width 0.4064) (layer "B.Cu") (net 15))
 (segment (start 166.2811 106.2736) (end 168.8211 106.2736) (width 0.4064) (layer "B.Cu") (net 15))
 (segment (start 135.8011 106.2736) (end 138.3411 106.2736) (width 0.4064) (layer "B.Cu") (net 15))
 (segment (start 151.0411 106.2736) (end 153.5811 106.2736) (width 0.4064) (layer "B.Cu") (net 15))
 (segment (start 153.5811 106.2736) (end 156.1211 106.2736) (width 0.4064) (layer "B.Cu") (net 15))
 (segment (start 138.3411 106.2736) (end 140.8811 106.2736) (width 0.4064) (layer "B.Cu") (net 15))
 (segment (start 143.4211 106.2736) (end 145.9611 106.2736) (width 0.4064) (layer "B.Cu") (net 15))
 (segment (start 158.6611 106.2736) (end 161.2011 106.2736) (width 0.4064) (layer "B.Cu") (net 15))
 (segment (start 128.1811 106.2736) (end 130.7211 106.2736) (width 0.4064) (layer "B.Cu") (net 15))
 (segment (start 163.7411 106.2736) (end 161.2011 106.2736) (width 0.4064) (layer "B.Cu") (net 15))
 (segment (start 156.1211 106.2736) (end 158.6611 106.2736) (width 0.4064) (layer "B.Cu") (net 15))
 (segment (start 133.3881 106.4006) (end 133.2611 106.2736) (width 0.4064) (layer "B.Cu") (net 15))
 (segment (start 135.8011 106.2736) (end 135.6741 106.4006) (width 0.4064) (layer "B.Cu") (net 15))
 (segment (start 134.5311 112.6236) (end 134.5311 115.1636) (width 0.4064) (layer "F.Cu") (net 16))
 (segment (start 129.4511 112.6236) (end 129.4511 115.1636) (width 0.4064) (layer "F.Cu") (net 17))
 (segment (start 139.6111 94.8436) (end 139.6111 97.3836) (width 0.4064) (layer "F.Cu") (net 28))
 (segment (start 142.1511 97.3836) (end 142.1511 94.8436) (width 0.4064) (layer "F.Cu") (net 27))
 (segment (start 135.4201 99.6696) (end 143.4211 99.6696) (width 0.4064) (layer "F.Cu") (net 26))
 (segment (start 134.5801 96.7486) (end 134.5801 98.8296) (width 0.4064) (layer "F.Cu") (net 26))
 (segment (start 144.6911 94.8436) (end 144.6911 97.3836) (width 0.4064) (layer "F.Cu") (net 26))
 (segment (start 143.4211 99.6696) (end 144.6911 98.3996) (width 0.4064) (layer "F.Cu") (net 26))
 (segment (start 144.6911 98.3996) (end 144.6911 97.3836) (width 0.4064) (layer "F.Cu") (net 26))
 (segment (start 134.5801 98.8296) (end 135.4201 99.6696) (width 0.4064) (layer "F.Cu") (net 26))
 (segment (start 165.0111 94.8436) (end 165.0111 97.3836) (width 0.4064) (layer "F.Cu") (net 19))
 (segment (start 154.8511 115.1636) (end 154.8511 112.6236) (width 0.4064) (layer "F.Cu") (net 8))
 (segment (start 157.3911 115.1636) (end 157.3911 112.6236) (width 0.4064) (layer "F.Cu") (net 7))
 (segment (start 159.9311 115.1636) (end 159.9311 112.6236) (width 0.4064) (layer "F.Cu") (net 6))
 (segment (start 162.4711 115.1636) (end 162.4711 112.6236) (width 0.4064) (layer "F.Cu") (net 5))
 (segment (start 165.0111 115.1636) (end 165.0111 112.6236) (width 0.4064) (layer "F.Cu") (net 4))
 (segment (start 167.5511 97.3836) (end 167.5511 94.8436) (width 0.4064) (layer "F.Cu") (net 18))
 (segment (start 129.4511 105.0036) (end 134.1501 105.0036) (width 0.254) (layer "F.Cu") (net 14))
 (segment (start 134.1501 105.0036) (end 134.5311 105.3846) (width 0.254) (layer "F.Cu") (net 14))
 (segment (start 128.1811 103.7336) (end 129.4511 105.0036) (width 0.254) (layer "F.Cu") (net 14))
 (segment (start 139.6111 112.6236) (end 139.6111 115.1636) (width 0.4064) (layer "F.Cu") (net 14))
 (segment (start 134.5311 107.5436) (end 139.6111 112.6236) (width 0.254) (layer "F.Cu") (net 14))
 (segment (start 134.5311 105.3846) (end 134.5311 107.5436) (width 0.254) (layer "F.Cu") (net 14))
 (segment (start 135.0391 105.0036) (end 133.7691 103.7336) (width 0.254) (layer "F.Cu") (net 13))
 (segment (start 139.3571 105.0036) (end 135.0391 105.0036) (width 0.254) (layer "F.Cu") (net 13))
 (segment (start 139.6619 105.3084) (end 139.6619 106.778613) (width 0.254) (layer "F.Cu") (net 13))
 (segment (start 139.6619 105.3084) (end 139.3571 105.0036) (width 0.254) (layer "F.Cu") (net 13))
 (segment (start 139.6619 106.778613) (end 142.1511 109.267813) (width 0.254) (layer "F.Cu") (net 13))
 (segment (start 142.1511 115.1636) (end 142.1511 112.6236) (width 0.4064) (layer "F.Cu") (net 13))
 (segment (start 133.7691 103.7336) (end 133.2611 103.7336) (width 0.254) (layer "F.Cu") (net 13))
 (segment (start 142.1511 109.267813) (end 142.1511 112.6236) (width 0.254) (layer "F.Cu") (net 13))
 (segment (start 144.6911 112.6236) (end 144.6911 115.1636) (width 0.4064) (layer "F.Cu") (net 12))
 (segment (start 142.2019 105.0544) (end 143.926112 105.0544) (width 0.254) (layer "F.Cu") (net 12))
 (segment (start 140.8811 103.7336) (end 142.2019 105.0544) (width 0.254) (layer "F.Cu") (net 12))
 (segment (start 143.926112 105.0544) (end 144.6911 105.819388) (width 0.254) (layer "F.Cu") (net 12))
 (segment (start 144.6911 105.819388) (end 144.6911 112.6236) (width 0.254) (layer "F.Cu") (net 12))
 (segment (start 147.2311 115.1636) (end 147.2311 112.6236) (width 0.4064) (layer "F.Cu") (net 11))
 (segment (start 145.9611 103.7336) (end 147.2311 105.0036) (width 0.254) (layer "F.Cu") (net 11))
 (segment (start 147.2311 105.0036) (end 147.2311 112.6236) (width 0.254) (layer "F.Cu") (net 11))
 (segment (start 149.7711 115.1636) (end 149.7711 112.7506) (width 0.4064) (layer "F.Cu") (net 10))
 (segment (start 149.7711 112.7506) (end 149.7711 112.6236) (width 0.4064) (layer "F.Cu") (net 10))
 (segment (start 148.5011 103.7336) (end 149.7711 105.0036) (width 0.254) (layer "F.Cu") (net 10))
 (segment (start 149.7711 105.0036) (end 149.7711 112.7506) (width 0.254) (layer "F.Cu") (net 10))
 (segment (start 151.0411 103.7336) (end 152.3111 105.0036) (width 0.254) (layer "F.Cu") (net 9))
 (segment (start 152.3111 115.1636) (end 152.3111 112.6236) (width 0.4064) (layer "F.Cu") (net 9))
 (segment (start 152.3111 105.0036) (end 152.3111 112.6236) (width 0.254) (layer "F.Cu") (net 9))
 (segment (start 152.3111 94.8436) (end 152.3111 97.3836) (width 0.4064) (layer "F.Cu") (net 23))
 (segment (start 152.3111 97.3836) (end 158.6611 103.7336) (width 0.254) (layer "F.Cu") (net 23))
 (segment (start 163.7411 103.7336) (end 165.0111 105.0036) (width 0.254) (layer "F.Cu") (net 1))
 (segment (start 157.3911 97.3836) (end 157.3911 94.8436) (width 0.4064) (layer "F.Cu") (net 1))
 (segment (start 157.3911 97.3836) (end 163.7411 103.7336) (width 0.254) (layer "F.Cu") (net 1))
 (segment (start 165.0111 105.0036) (end 165.0111 109.4096) (width 0.254) (layer "F.Cu") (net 1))
 (segment (start 165.0111 109.4096) (end 164.0561 110.4646) (width 0.254) (layer "F.Cu") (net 1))
 (segment (start 159.9311 94.8436) (end 159.9311 97.3836) (width 0.4064) (layer "F.Cu") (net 21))
 (segment (start 159.9311 97.3836) (end 166.2811 103.7336) (width 0.254) (layer "F.Cu") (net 21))
 (segment (start 168.8211 103.7336) (end 162.4711 97.3836) (width 0.254) (layer "F.Cu") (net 20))
 (segment (start 162.4711 97.3836) (end 162.4711 94.8436) (width 0.4064) (layer "F.Cu") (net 20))
 (segment (start 147.2311 94.8436) (end 147.2311 97.3836) (width 0.4064) (layer "F.Cu") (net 25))
 (segment (start 147.2311 97.3836) (end 153.5811 103.7336) (width 0.254) (layer "F.Cu") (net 25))
 (segment (start 149.7711 97.3836) (end 156.1211 103.7336) (width 0.254) (layer "F.Cu") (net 24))
 (segment (start 149.7711 94.8436) (end 149.7711 97.3836) (width 0.4064) (layer "F.Cu") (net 24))
 (segment (start 154.8511 97.3836) (end 161.2011 103.7336) (width 0.254) (layer "F.Cu") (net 22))
 (segment (start 154.8511 94.8436) (end 154.8511 97.3836) (width 0.4064) (layer "F.Cu") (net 22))
 (segment (start 162.1561 110.4646) (end 160.1851 110.4646) (width 0.254) (layer "F.Cu") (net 2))
 (segment (start 131.9911 115.1636) (end 131.9911 112.6236) (width 0.4064) (layer "F.Cu") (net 2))
 (via (at 160.1851 110.4646) (size 0.9064) (drill 0.5) (layers "F.Cu" "B.Cu") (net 2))
 (segment (start 132.6261 110.4646) (end 131.9911 111.0996) (width 0.254) (layer "B.Cu") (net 2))
 (segment (start 160.1851 110.4646) (end 132.6261 110.4646) (width 0.254) (layer "B.Cu") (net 2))
 (segment (start 131.9911 111.0996) (end 131.9911 112.6236) (width 0.254) (layer "B.Cu") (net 2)))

